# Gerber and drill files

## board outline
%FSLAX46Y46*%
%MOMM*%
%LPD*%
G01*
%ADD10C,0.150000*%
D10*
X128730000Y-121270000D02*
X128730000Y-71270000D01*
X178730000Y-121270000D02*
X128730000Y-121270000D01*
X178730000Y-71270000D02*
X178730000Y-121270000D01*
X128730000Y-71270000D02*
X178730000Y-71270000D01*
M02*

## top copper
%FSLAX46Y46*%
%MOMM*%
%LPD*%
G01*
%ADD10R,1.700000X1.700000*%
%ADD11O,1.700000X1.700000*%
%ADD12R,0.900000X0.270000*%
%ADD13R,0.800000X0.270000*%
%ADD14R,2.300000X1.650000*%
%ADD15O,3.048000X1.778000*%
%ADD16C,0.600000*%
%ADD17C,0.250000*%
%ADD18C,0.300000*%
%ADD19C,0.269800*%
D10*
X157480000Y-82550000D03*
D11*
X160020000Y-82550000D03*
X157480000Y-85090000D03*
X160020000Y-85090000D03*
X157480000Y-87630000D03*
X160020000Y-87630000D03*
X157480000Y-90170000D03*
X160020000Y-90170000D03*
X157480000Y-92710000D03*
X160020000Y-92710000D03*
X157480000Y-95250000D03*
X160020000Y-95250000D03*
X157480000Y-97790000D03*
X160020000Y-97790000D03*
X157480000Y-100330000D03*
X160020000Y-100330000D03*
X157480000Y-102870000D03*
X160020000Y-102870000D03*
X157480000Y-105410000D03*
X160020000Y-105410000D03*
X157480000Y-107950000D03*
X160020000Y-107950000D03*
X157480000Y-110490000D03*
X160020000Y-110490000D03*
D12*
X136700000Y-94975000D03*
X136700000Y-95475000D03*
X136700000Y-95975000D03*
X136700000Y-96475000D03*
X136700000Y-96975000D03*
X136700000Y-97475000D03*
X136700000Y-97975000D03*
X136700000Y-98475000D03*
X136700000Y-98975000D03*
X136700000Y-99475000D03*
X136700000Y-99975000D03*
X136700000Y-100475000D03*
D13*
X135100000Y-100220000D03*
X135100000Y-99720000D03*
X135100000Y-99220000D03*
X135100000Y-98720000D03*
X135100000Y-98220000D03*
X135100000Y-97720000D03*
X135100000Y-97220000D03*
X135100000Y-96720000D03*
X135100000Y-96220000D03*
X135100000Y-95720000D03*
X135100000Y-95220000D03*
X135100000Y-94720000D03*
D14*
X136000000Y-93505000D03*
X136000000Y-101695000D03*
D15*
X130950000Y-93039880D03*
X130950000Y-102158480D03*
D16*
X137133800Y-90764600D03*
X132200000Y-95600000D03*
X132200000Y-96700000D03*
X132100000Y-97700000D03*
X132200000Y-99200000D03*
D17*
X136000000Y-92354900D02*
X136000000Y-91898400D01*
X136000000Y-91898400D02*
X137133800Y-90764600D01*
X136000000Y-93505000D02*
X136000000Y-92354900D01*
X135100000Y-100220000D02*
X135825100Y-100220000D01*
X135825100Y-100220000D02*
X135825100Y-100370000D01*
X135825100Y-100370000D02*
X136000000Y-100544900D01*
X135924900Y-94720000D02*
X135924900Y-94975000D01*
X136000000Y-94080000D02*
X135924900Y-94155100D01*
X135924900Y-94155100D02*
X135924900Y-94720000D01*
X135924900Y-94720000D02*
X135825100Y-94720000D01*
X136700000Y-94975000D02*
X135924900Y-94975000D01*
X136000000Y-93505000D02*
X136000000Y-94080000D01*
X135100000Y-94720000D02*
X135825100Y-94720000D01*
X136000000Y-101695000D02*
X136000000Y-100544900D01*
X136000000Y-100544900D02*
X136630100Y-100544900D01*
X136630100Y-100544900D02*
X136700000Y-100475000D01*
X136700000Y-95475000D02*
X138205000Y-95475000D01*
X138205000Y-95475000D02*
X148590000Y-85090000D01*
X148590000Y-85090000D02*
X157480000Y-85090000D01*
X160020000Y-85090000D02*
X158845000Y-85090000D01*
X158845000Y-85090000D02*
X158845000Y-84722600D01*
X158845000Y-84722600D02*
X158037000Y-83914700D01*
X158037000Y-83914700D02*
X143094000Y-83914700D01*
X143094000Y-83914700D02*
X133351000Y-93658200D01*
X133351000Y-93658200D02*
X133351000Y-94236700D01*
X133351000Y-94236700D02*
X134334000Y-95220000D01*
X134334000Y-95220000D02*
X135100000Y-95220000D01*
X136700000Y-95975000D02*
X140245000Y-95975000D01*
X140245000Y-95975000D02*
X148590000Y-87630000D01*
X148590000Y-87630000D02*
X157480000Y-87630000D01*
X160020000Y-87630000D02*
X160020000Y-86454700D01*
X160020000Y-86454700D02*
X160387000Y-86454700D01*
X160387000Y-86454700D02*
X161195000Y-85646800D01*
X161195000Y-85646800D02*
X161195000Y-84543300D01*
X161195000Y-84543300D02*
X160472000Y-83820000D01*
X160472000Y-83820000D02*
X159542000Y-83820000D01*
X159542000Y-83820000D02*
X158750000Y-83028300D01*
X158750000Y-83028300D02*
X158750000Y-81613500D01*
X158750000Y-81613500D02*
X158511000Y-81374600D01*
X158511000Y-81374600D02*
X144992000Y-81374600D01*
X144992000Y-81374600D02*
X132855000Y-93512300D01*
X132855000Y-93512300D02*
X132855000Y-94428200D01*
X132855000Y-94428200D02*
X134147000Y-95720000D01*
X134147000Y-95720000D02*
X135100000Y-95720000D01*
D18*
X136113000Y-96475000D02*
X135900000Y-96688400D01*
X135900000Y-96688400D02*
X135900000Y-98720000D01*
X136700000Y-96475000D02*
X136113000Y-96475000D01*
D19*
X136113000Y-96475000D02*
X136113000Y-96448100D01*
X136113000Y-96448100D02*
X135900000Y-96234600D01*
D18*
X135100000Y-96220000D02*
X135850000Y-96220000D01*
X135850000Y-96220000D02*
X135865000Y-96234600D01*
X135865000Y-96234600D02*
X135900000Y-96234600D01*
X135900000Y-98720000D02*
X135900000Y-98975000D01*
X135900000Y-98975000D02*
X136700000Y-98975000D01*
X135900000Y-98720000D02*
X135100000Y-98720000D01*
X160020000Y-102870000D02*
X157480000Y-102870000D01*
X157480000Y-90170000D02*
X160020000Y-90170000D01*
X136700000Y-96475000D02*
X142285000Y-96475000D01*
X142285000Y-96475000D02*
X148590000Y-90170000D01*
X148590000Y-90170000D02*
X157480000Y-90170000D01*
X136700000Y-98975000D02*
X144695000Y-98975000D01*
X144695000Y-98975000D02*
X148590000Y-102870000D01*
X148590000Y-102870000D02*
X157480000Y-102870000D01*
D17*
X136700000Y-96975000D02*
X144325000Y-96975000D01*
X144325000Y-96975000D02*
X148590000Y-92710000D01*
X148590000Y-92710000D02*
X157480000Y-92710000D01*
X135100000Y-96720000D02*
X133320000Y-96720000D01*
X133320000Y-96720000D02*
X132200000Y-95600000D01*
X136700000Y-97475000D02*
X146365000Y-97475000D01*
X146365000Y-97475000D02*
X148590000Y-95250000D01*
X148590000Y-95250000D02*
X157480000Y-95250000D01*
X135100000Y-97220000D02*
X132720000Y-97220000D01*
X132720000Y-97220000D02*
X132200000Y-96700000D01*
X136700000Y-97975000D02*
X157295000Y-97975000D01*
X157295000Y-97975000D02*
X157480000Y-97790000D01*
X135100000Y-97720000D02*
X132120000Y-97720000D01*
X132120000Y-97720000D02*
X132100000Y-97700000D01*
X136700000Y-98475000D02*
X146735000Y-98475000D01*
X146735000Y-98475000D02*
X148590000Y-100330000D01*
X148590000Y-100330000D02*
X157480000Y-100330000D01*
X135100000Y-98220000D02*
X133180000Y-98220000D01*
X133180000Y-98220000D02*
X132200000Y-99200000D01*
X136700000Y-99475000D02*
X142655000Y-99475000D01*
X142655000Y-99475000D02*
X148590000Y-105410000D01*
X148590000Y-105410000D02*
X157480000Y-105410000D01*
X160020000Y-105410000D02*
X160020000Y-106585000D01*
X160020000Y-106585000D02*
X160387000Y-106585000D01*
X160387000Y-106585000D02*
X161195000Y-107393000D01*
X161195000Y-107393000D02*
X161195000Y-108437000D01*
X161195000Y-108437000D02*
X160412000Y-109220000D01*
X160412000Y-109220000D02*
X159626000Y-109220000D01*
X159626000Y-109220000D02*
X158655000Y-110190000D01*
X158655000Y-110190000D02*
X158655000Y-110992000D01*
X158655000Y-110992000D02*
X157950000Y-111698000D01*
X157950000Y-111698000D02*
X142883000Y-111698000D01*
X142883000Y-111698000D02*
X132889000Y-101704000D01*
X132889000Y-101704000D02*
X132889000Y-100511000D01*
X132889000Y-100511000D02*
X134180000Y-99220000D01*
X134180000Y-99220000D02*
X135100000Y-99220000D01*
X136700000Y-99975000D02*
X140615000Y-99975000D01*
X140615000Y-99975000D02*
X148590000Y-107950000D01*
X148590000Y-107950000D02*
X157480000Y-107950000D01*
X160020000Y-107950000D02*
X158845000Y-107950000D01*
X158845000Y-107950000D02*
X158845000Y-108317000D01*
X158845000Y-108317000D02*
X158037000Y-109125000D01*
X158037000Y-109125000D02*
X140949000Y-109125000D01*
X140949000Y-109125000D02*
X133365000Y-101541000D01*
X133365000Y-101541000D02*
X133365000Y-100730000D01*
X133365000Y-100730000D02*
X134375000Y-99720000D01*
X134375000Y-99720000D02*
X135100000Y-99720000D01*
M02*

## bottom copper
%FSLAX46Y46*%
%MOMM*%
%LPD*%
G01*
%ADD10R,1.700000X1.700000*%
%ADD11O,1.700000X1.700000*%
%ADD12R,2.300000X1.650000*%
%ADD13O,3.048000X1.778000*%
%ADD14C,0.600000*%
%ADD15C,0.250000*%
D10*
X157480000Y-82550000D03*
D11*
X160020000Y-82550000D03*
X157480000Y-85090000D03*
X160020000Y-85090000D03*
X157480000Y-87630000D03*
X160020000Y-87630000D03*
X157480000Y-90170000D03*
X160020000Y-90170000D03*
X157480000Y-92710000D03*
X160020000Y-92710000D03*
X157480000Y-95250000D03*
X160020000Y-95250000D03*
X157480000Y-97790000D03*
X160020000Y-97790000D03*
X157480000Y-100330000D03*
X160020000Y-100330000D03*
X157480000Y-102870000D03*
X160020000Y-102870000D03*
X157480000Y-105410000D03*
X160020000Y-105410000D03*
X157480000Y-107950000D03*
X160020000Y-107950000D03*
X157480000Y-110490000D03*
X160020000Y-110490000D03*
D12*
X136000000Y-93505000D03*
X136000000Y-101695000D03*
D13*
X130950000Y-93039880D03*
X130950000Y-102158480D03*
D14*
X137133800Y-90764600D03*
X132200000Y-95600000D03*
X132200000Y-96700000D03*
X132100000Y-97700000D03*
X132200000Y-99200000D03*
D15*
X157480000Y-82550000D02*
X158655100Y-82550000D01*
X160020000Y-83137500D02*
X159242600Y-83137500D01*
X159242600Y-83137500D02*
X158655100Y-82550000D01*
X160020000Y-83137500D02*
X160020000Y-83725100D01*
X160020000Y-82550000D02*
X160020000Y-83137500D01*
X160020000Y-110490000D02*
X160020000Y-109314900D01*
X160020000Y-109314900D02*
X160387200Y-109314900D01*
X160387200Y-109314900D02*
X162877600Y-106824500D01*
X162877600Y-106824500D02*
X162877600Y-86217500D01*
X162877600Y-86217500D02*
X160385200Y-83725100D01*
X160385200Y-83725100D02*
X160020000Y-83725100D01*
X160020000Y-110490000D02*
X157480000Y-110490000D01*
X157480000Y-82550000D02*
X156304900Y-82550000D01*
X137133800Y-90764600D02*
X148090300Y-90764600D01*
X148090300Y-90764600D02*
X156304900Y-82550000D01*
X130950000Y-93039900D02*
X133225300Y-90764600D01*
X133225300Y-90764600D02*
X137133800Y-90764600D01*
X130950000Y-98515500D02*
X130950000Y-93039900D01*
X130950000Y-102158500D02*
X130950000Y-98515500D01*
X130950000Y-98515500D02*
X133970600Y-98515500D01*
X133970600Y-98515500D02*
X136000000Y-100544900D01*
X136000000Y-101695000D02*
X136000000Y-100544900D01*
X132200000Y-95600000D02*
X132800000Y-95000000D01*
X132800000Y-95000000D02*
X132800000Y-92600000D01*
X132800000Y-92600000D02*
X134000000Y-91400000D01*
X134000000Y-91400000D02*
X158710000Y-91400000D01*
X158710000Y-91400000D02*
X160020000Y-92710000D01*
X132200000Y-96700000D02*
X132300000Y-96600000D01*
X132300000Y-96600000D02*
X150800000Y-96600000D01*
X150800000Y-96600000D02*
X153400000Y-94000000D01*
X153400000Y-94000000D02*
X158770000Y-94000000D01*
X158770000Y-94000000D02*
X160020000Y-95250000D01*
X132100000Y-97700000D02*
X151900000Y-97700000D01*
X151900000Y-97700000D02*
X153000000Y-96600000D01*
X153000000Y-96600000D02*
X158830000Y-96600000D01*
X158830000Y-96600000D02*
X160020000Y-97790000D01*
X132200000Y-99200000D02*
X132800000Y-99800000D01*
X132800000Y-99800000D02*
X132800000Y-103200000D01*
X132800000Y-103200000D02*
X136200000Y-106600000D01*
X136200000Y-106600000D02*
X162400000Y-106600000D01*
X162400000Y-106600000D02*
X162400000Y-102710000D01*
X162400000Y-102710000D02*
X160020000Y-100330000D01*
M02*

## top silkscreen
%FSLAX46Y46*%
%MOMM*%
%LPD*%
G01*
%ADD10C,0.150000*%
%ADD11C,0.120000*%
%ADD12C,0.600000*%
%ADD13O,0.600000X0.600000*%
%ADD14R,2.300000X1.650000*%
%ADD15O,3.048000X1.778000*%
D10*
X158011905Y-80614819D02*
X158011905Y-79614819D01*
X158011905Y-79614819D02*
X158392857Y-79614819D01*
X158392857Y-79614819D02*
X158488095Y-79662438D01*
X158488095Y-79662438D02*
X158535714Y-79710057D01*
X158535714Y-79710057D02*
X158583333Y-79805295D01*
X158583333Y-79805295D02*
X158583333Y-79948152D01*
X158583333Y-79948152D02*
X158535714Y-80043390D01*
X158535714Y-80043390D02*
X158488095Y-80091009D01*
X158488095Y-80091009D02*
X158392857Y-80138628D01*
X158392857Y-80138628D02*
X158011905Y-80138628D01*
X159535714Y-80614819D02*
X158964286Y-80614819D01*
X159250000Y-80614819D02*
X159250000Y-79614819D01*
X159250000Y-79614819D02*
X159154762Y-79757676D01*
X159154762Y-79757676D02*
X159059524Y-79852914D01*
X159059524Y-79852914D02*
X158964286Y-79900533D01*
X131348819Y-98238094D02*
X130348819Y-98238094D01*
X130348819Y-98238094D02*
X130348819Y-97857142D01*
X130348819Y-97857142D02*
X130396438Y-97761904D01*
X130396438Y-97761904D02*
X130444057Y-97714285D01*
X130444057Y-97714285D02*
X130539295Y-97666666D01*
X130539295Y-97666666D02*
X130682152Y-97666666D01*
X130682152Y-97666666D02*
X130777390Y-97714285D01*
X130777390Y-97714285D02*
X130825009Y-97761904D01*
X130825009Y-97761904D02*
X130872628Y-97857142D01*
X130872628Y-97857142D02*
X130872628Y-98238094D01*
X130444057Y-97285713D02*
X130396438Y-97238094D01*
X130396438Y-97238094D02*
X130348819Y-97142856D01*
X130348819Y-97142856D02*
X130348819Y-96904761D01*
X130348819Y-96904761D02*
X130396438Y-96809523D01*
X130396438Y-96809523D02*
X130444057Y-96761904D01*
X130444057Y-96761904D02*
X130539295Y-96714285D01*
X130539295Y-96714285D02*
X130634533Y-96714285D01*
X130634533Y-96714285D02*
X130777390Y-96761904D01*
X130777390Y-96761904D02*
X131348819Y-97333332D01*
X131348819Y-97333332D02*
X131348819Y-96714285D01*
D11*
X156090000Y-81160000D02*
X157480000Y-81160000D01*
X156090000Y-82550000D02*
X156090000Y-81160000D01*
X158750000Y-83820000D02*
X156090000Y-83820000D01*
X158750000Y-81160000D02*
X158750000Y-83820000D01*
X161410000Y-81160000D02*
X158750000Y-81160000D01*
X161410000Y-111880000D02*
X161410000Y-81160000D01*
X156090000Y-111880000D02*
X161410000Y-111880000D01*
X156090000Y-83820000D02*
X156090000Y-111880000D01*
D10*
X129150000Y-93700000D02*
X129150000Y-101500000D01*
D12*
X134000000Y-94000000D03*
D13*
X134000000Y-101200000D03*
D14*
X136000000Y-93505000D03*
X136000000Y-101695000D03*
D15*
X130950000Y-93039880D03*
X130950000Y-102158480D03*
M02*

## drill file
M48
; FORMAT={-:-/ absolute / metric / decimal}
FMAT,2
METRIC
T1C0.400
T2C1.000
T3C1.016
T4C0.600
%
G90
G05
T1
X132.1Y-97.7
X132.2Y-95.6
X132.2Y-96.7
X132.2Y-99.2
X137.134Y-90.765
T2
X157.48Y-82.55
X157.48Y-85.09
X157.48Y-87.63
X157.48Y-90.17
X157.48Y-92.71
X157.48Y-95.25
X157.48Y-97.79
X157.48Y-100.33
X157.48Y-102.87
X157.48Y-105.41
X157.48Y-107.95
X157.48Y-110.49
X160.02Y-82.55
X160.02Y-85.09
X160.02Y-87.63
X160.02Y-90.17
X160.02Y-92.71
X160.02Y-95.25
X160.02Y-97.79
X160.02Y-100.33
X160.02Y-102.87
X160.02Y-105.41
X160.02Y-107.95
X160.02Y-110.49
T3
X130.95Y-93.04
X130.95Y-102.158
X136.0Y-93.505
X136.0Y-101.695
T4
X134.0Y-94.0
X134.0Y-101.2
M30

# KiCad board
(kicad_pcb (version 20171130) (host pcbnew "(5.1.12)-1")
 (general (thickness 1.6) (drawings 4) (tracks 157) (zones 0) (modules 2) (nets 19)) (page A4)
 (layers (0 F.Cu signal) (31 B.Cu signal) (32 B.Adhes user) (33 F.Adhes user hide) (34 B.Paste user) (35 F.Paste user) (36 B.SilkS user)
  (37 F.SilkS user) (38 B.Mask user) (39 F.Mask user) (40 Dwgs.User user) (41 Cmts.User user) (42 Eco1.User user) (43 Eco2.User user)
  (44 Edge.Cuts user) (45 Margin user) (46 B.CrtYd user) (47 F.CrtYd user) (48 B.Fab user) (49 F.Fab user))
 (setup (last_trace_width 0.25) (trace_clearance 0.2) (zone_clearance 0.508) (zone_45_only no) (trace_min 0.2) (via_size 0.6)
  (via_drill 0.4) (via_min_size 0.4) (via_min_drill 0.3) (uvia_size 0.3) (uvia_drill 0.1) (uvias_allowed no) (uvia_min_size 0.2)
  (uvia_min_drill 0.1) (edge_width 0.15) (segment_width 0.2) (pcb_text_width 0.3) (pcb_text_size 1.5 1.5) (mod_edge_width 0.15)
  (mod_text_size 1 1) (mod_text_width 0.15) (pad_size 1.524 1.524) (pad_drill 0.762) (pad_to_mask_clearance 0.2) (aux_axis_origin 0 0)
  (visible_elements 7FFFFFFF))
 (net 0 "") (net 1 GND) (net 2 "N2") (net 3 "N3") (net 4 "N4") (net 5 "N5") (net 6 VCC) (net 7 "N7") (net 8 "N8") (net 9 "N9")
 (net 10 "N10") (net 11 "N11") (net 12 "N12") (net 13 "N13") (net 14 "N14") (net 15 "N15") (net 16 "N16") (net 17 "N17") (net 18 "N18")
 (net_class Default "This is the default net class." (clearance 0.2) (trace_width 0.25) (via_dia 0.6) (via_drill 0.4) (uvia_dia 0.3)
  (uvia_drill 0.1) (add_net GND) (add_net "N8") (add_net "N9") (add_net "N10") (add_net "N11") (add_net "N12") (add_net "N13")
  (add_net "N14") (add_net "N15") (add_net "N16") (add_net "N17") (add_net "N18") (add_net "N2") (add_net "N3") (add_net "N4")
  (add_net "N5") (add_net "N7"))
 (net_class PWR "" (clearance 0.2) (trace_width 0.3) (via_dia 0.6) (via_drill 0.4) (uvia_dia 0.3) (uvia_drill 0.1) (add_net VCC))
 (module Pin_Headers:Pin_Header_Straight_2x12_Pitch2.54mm (layer F.Cu) (at 157.48 82.55)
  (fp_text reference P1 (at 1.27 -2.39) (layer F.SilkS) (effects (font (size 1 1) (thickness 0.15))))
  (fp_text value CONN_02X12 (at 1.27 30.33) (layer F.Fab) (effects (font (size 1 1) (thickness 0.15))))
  (fp_line (start -1.39 -1.39) (end 0 -1.39) (layer F.SilkS) (width 0.12))
  (fp_line (start -1.39 0) (end -1.39 -1.39) (layer F.SilkS) (width 0.12))
  (fp_line (start 1.27 1.27) (end -1.39 1.27) (layer F.SilkS) (width 0.12))
  (fp_line (start 1.27 -1.39) (end 1.27 1.27) (layer F.SilkS) (width 0.12))
  (fp_line (start 3.93 -1.39) (end 1.27 -1.39) (layer F.SilkS) (width 0.12))
  (fp_line (start 3.93 29.33) (end 3.93 -1.39) (layer F.SilkS) (width 0.12))
  (fp_line (start -1.39 29.33) (end 3.93 29.33) (layer F.SilkS) (width 0.12))
  (fp_line (start -1.39 1.27) (end -1.39 29.33) (layer F.SilkS) (width 0.12))
  (pad 1 thru_hole rect (at 0 0) (size 1.7 1.7) (drill 1) (layers *.Cu *.Mask) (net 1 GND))
  (pad 2 thru_hole oval (at 2.54 0) (size 1.7 1.7) (drill 1) (layers *.Cu *.Mask) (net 1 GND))
  (pad 3 thru_hole oval (at 0 2.54) (size 1.7 1.7) (drill 1) (layers *.Cu *.Mask) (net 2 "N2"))
  (pad 4 thru_hole oval (at 2.54 2.54) (size 1.7 1.7) (drill 1) (layers *.Cu *.Mask) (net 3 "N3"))
  (pad 5 thru_hole oval (at 0 5.08) (size 1.7 1.7) (drill 1) (layers *.Cu *.Mask) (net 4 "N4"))
  (pad 6 thru_hole oval (at 2.54 5.08) (size 1.7 1.7) (drill 1) (layers *.Cu *.Mask) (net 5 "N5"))
  (pad 7 thru_hole oval (at 0 7.62) (size 1.7 1.7) (drill 1) (layers *.Cu *.Mask) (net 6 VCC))
  (pad 8 thru_hole oval (at 2.54 7.62) (size 1.7 1.7) (drill 1) (layers *.Cu *.Mask) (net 6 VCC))
  (pad 9 thru_hole oval (at 0 10.16) (size 1.7 1.7) (drill 1) (layers *.Cu *.Mask) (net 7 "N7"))
  (pad 10 thru_hole oval (at 2.54 10.16) (size 1.7 1.7) (drill 1) (layers *.Cu *.Mask) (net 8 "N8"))
  (pad 11 thru_hole oval (at 0 12.7) (size 1.7 1.7) (drill 1) (layers *.Cu *.Mask) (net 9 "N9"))
  (pad 12 thru_hole oval (at 2.54 12.7) (size 1.7 1.7) (drill 1) (layers *.Cu *.Mask) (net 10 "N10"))
  (pad 13 thru_hole oval (at 0 15.24) (size 1.7 1.7) (drill 1) (layers *.Cu *.Mask) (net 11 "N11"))
  (pad 14 thru_hole oval (at 2.54 15.24) (size 1.7 1.7) (drill 1) (layers *.Cu *.Mask) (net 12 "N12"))
  (pad 15 thru_hole oval (at 0 17.78) (size 1.7 1.7) (drill 1) (layers *.Cu *.Mask) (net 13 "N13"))
  (pad 16 thru_hole oval (at 2.54 17.78) (size 1.7 1.7) (drill 1) (layers *.Cu *.Mask) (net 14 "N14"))
  (pad 17 thru_hole oval (at 0 20.32) (size 1.7 1.7) (drill 1) (layers *.Cu *.Mask) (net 6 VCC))
  (pad 18 thru_hole oval (at 2.54 20.32) (size 1.7 1.7) (drill 1) (layers *.Cu *.Mask) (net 6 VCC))
  (pad 19 thru_hole oval (at 0 22.86) (size 1.7 1.7) (drill 1) (layers *.Cu *.Mask) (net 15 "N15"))
  (pad 20 thru_hole oval (at 2.54 22.86) (size 1.7 1.7) (drill 1) (layers *.Cu *.Mask) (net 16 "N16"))
  (pad 21 thru_hole oval (at 0 25.4) (size 1.7 1.7) (drill 1) (layers *.Cu *.Mask) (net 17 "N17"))
  (pad 22 thru_hole oval (at 2.54 25.4) (size 1.7 1.7) (drill 1) (layers *.Cu *.Mask) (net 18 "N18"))
  (pad 23 thru_hole oval (at 0 27.94) (size 1.7 1.7) (drill 1) (layers *.Cu *.Mask) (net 1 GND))
  (pad 24 thru_hole oval (at 2.54 27.94) (size 1.7 1.7) (drill 1) (layers *.Cu *.Mask) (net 1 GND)))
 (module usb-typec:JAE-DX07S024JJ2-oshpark (layer F.Cu) (at 134 94 270)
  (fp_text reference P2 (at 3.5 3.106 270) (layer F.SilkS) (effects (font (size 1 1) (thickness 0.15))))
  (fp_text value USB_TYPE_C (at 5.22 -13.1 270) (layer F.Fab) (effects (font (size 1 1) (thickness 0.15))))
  (fp_line (start -0.3 4.85) (end 7.5 4.85) (layer F.SilkS) (width 0.15))
  (pad A1 smd rect (at 0.975 -2.7 270) (size 0.27 0.9) (layers F.Cu F.Paste F.Mask) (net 1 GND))
  (pad A2 smd rect (at 1.475 -2.7 270) (size 0.27 0.9) (layers F.Cu F.Paste F.Mask) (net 2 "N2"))
  (pad A3 smd rect (at 1.975 -2.7 270) (size 0.27 0.9) (layers F.Cu F.Paste F.Mask) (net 4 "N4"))
  (pad A4 smd rect (at 2.475 -2.7 270) (size 0.27 0.9) (layers F.Cu F.Paste F.Mask) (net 6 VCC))
  (pad A5 smd rect (at 2.975 -2.7 270) (size 0.27 0.9) (layers F.Cu F.Paste F.Mask) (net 7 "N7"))
  (pad A6 smd rect (at 3.475 -2.7 270) (size 0.27 0.9) (layers F.Cu F.Paste F.Mask) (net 9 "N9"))
  (pad A7 smd rect (at 3.975 -2.7 270) (size 0.27 0.9) (layers F.Cu F.Paste F.Mask) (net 11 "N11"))
  (pad A8 smd rect (at 4.475 -2.7 270) (size 0.27 0.9) (layers F.Cu F.Paste F.Mask) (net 13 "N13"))
  (pad A9 smd rect (at 4.975 -2.7 270) (size 0.27 0.9) (layers F.Cu F.Paste F.Mask) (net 6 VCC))
  (pad A10 smd rect (at 5.475 -2.7 270) (size 0.27 0.9) (layers F.Cu F.Paste F.Mask) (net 15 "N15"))
  (pad A11 smd rect (at 5.975 -2.7 270) (size 0.27 0.9) (layers F.Cu F.Paste F.Mask) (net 17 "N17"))
  (pad A12 smd rect (at 6.475 -2.7 270) (size 0.27 0.9) (layers F.Cu F.Paste F.Mask) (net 1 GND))
  (pad B1 smd rect (at 6.22 -1.1 270) (size 0.27 0.8) (layers F.Cu F.Paste F.Mask) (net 1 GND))
  (pad B2 smd rect (at 5.72 -1.1 270) (size 0.27 0.8) (layers F.Cu F.Paste F.Mask) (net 18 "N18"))
  (pad B3 smd rect (at 5.22 -1.1 270) (size 0.27 0.8) (layers F.Cu F.Paste F.Mask) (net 16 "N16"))
  (pad B4 smd rect (at 4.72 -1.1 270) (size 0.27 0.8) (layers F.Cu F.Paste F.Mask) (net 6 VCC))
  (pad B5 smd rect (at 4.22 -1.1 270) (size 0.27 0.8) (layers F.Cu F.Paste F.Mask) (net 14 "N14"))
  (pad B6 smd rect (at 3.72 -1.1 270) (size 0.27 0.8) (layers F.Cu F.Paste F.Mask) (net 12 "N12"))
  (pad B7 smd rect (at 3.22 -1.1 270) (size 0.27 0.8) (layers F.Cu F.Paste F.Mask) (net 10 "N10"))
  (pad B8 smd rect (at 2.72 -1.1 270) (size 0.27 0.8) (layers F.Cu F.Paste F.Mask) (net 8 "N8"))
  (pad B9 smd rect (at 2.22 -1.1 270) (size 0.27 0.8) (layers F.Cu F.Paste F.Mask) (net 6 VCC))
  (pad B10 smd rect (at 1.72 -1.1 270) (size 0.27 0.8) (layers F.Cu F.Paste F.Mask) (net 5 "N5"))
  (pad B11 smd rect (at 1.22 -1.1 270) (size 0.27 0.8) (layers F.Cu F.Paste F.Mask) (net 3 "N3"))
  (pad B12 smd rect (at 0.72 -1.1 270) (size 0.27 0.8) (layers F.Cu F.Paste F.Mask) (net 1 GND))
  (pad "" np_thru_hole circle (at 0 0 270) (size 0.6 0.6) (drill 0.6) (layers *.Cu *.Mask F.SilkS))
  (pad "" np_thru_hole oval (at 7.2 0 270) (size 0.6 0.6) (drill 0.6) (layers *.Cu *.Mask F.SilkS))
  (pad 0 thru_hole rect (at -0.495 -2 270) (size 1.65 2.3) (drill 1.016) (layers *.Cu *.Mask F.SilkS) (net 1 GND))
  (pad 0 thru_hole rect (at 7.695 -2 270) (size 1.65 2.3) (drill 1.016) (layers *.Cu *.Mask F.SilkS) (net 1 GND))
  (pad 0 thru_hole oval (at -0.96012 3.05 270) (size 1.778 3.048) (drill 1.016) (layers *.Cu *.Mask F.SilkS) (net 1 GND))
  (pad 0 thru_hole oval (at 8.15848 3.05 270) (size 1.778 3.048) (drill 1.016) (layers *.Cu *.Mask F.SilkS) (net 1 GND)))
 (gr_line (start 128.73 121.27) (end 128.73 71.27) (angle 90) (layer Edge.Cuts) (width 0.15))
 (gr_line (start 178.73 121.27) (end 128.73 121.27) (angle 90) (layer Edge.Cuts) (width 0.15))
 (gr_line (start 178.73 71.27) (end 178.73 121.27) (angle 90) (layer Edge.Cuts) (width 0.15))
 (gr_line (start 128.73 71.27) (end 178.73 71.27) (angle 90) (layer Edge.Cuts) (width 0.15))
 (segment (start 157.48 82.55) (end 158.6551 82.55) (width 0.25) (layer B.Cu) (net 1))
 (segment (start 160.02 83.1375) (end 159.2426 83.1375) (width 0.25) (layer B.Cu) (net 1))
 (segment (start 159.2426 83.1375) (end 158.6551 82.55) (width 0.25) (layer B.Cu) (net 1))
 (segment (start 160.02 83.1375) (end 160.02 83.7251) (width 0.25) (layer B.Cu) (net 1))
 (segment (start 160.02 82.55) (end 160.02 83.1375) (width 0.25) (layer B.Cu) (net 1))
 (segment (start 160.02 110.49) (end 160.02 109.3149) (width 0.25) (layer B.Cu) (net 1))
 (segment (start 160.02 109.3149) (end 160.3872 109.3149) (width 0.25) (layer B.Cu) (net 1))
 (segment (start 160.3872 109.3149) (end 162.8776 106.8245) (width 0.25) (layer B.Cu) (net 1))
 (segment (start 162.8776 106.8245) (end 162.8776 86.2175) (width 0.25) (layer B.Cu) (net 1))
 (segment (start 162.8776 86.2175) (end 160.3852 83.7251) (width 0.25) (layer B.Cu) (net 1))
 (segment (start 160.3852 83.7251) (end 160.02 83.7251) (width 0.25) (layer B.Cu) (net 1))
 (segment (start 160.02 110.49) (end 157.48 110.49) (width 0.25) (layer B.Cu) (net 1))
 (segment (start 157.48 82.55) (end 156.3049 82.55) (width 0.25) (layer B.Cu) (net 1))
 (segment (start 137.1338 90.7646) (end 148.0903 90.7646) (width 0.25) (layer B.Cu) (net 1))
 (segment (start 148.0903 90.7646) (end 156.3049 82.55) (width 0.25) (layer B.Cu) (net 1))
 (segment (start 130.95 93.0399) (end 133.2253 90.7646) (width 0.25) (layer B.Cu) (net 1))
 (segment (start 133.2253 90.7646) (end 137.1338 90.7646) (width 0.25) (layer B.Cu) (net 1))
 (segment (start 136 92.3549) (end 136 91.8984) (width 0.25) (layer F.Cu) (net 1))
 (segment (start 136 91.8984) (end 137.1338 90.7646) (width 0.25) (layer F.Cu) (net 1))
 (segment (start 136 93.505) (end 136 92.3549) (width 0.25) (layer F.Cu) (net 1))
 (segment (start 130.95 98.5155) (end 130.95 93.0399) (width 0.25) (layer B.Cu) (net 1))
 (segment (start 135.1 100.22) (end 135.8251 100.22) (width 0.25) (layer F.Cu) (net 1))
 (segment (start 135.8251 100.22) (end 135.8251 100.37) (width 0.25) (layer F.Cu) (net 1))
 (segment (start 135.8251 100.37) (end 136 100.5449) (width 0.25) (layer F.Cu) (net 1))
 (segment (start 135.9249 94.72) (end 135.9249 94.975) (width 0.25) (layer F.Cu) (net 1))
 (segment (start 136 94.08) (end 135.9249 94.1551) (width 0.25) (layer F.Cu) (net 1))
 (segment (start 135.9249 94.1551) (end 135.9249 94.72) (width 0.25) (layer F.Cu) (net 1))
 (segment (start 135.9249 94.72) (end 135.8251 94.72) (width 0.25) (layer F.Cu) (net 1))
 (segment (start 136.7 94.975) (end 135.9249 94.975) (width 0.25) (layer F.Cu) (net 1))
 (segment (start 136 93.505) (end 136 94.08) (width 0.25) (layer F.Cu) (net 1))
 (segment (start 135.1 94.72) (end 135.8251 94.72) (width 0.25) (layer F.Cu) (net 1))
 (segment (start 136 101.695) (end 136 100.5449) (width 0.25) (layer F.Cu) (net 1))
 (segment (start 136 100.5449) (end 136.6301 100.5449) (width 0.25) (layer F.Cu) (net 1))
 (segment (start 136.6301 100.5449) (end 136.7 100.475) (width 0.25) (layer F.Cu) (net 1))
 (segment (start 130.95 102.1585) (end 130.95 98.5155) (width 0.25) (layer B.Cu) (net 1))
 (segment (start 130.95 98.5155) (end 133.9706 98.5155) (width 0.25) (layer B.Cu) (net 1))
 (segment (start 133.9706 98.5155) (end 136 100.5449) (width 0.25) (layer B.Cu) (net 1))
 (segment (start 136 101.695) (end 136 100.5449) (width 0.25) (layer B.Cu) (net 1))
 (via (at 137.1338 90.7646) (size 0.6) (layers F.Cu B.Cu) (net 1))
 (segment (start 136.7 95.475) (end 138.205 95.475) (width 0.25) (layer F.Cu) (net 2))
 (segment (start 138.205 95.475) (end 148.59 85.09) (width 0.25) (layer F.Cu) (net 2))
 (segment (start 148.59 85.09) (end 157.48 85.09) (width 0.25) (layer F.Cu) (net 2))
 (segment (start 160.02 85.09) (end 158.845 85.09) (width 0.25) (layer F.Cu) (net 3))
 (segment (start 158.845 85.09) (end 158.845 84.7226) (width 0.25) (layer F.Cu) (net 3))
 (segment (start 158.845 84.7226) (end 158.037 83.9147) (width 0.25) (layer F.Cu) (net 3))
 (segment (start 158.037 83.9147) (end 143.094 83.9147) (width 0.25) (layer F.Cu) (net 3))
 (segment (start 143.094 83.9147) (end 133.351 93.6582) (width 0.25) (layer F.Cu) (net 3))
 (segment (start 133.351 93.6582) (end 133.351 94.2367) (width 0.25) (layer F.Cu) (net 3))
 (segment (start 133.351 94.2367) (end 134.334 95.22) (width 0.25) (layer F.Cu) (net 3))
 (segment (start 134.334 95.22) (end 135.1 95.22) (width 0.25) (layer F.Cu) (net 3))
 (segment (start 136.7 95.975) (end 140.245 95.975) (width 0.25) (layer F.Cu) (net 4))
 (segment (start 140.245 95.975) (end 148.59 87.63) (width 0.25) (layer F.Cu) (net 4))
 (segment (start 148.59 87.63) (end 157.48 87.63) (width 0.25) (layer F.Cu) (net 4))
 (segment (start 160.02 87.63) (end 160.02 86.4547) (width 0.25) (layer F.Cu) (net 5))
 (segment (start 160.02 86.4547) (end 160.387 86.4547) (width 0.25) (layer F.Cu) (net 5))
 (segment (start 160.387 86.4547) (end 161.195 85.6468) (width 0.25) (layer F.Cu) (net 5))
 (segment (start 161.195 85.6468) (end 161.195 84.5433) (width 0.25) (layer F.Cu) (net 5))
 (segment (start 161.195 84.5433) (end 160.472 83.82) (width 0.25) (layer F.Cu) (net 5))
 (segment (start 160.472 83.82) (end 159.542 83.82) (width 0.25) (layer F.Cu) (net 5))
 (segment (start 159.542 83.82) (end 158.75 83.0283) (width 0.25) (layer F.Cu) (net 5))
 (segment (start 158.75 83.0283) (end 158.75 81.6135) (width 0.25) (layer F.Cu) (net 5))
 (segment (start 158.75 81.6135) (end 158.511 81.3746) (width 0.25) (layer F.Cu) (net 5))
 (segment (start 158.511 81.3746) (end 144.992 81.3746) (width 0.25) (layer F.Cu) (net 5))
 (segment (start 144.992 81.3746) (end 132.855 93.5123) (width 0.25) (layer F.Cu) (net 5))
 (segment (start 132.855 93.5123) (end 132.855 94.4282) (width 0.25) (layer F.Cu) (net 5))
 (segment (start 132.855 94.4282) (end 134.147 95.72) (width 0.25) (layer F.Cu) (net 5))
 (segment (start 134.147 95.72) (end 135.1 95.72) (width 0.25) (layer F.Cu) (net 5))
 (segment (start 136.113 96.475) (end 135.9 96.6884) (width 0.3) (layer F.Cu) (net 6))
 (segment (start 135.9 96.6884) (end 135.9 98.72) (width 0.3) (layer F.Cu) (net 6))
 (segment (start 136.7 96.475) (end 136.113 96.475) (width 0.3) (layer F.Cu) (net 6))
 (segment (start 136.113 96.475) (end 136.113 96.4481) (width 0.2698) (layer F.Cu) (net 6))
 (segment (start 136.113 96.4481) (end 135.9 96.2346) (width 0.2698) (layer F.Cu) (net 6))
 (segment (start 135.1 96.22) (end 135.85 96.22) (width 0.3) (layer F.Cu) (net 6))
 (segment (start 135.85 96.22) (end 135.865 96.2346) (width 0.3) (layer F.Cu) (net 6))
 (segment (start 135.865 96.2346) (end 135.9 96.2346) (width 0.3) (layer F.Cu) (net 6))
 (segment (start 135.9 98.72) (end 135.9 98.975) (width 0.3) (layer F.Cu) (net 6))
 (segment (start 135.9 98.975) (end 136.7 98.975) (width 0.3) (layer F.Cu) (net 6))
 (segment (start 135.9 98.72) (end 135.1 98.72) (width 0.3) (layer F.Cu) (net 6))
 (segment (start 160.02 102.87) (end 157.48 102.87) (width 0.3) (layer F.Cu) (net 6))
 (segment (start 157.48 90.17) (end 160.02 90.17) (width 0.3) (layer F.Cu) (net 6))
 (segment (start 136.7 96.475) (end 142.285 96.475) (width 0.3) (layer F.Cu) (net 6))
 (segment (start 142.285 96.475) (end 148.59 90.17) (width 0.3) (layer F.Cu) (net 6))
 (segment (start 148.59 90.17) (end 157.48 90.17) (width 0.3) (layer F.Cu) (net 6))
 (segment (start 136.7 98.975) (end 144.695 98.975) (width 0.3) (layer F.Cu) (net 6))
 (segment (start 144.695 98.975) (end 148.59 102.87) (width 0.3) (layer F.Cu) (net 6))
 (segment (start 148.59 102.87) (end 157.48 102.87) (width 0.3) (layer F.Cu) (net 6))
 (segment (start 136.7 96.975) (end 144.325 96.975) (width 0.25) (layer F.Cu) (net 7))
 (segment (start 144.325 96.975) (end 148.59 92.71) (width 0.25) (layer F.Cu) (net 7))
 (segment (start 148.59 92.71) (end 157.48 92.71) (width 0.25) (layer F.Cu) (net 7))
 (segment (start 135.1 96.72) (end 133.32 96.72) (width 0.25) (layer F.Cu) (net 8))
 (segment (start 133.32 96.72) (end 132.2 95.6) (width 0.25) (layer F.Cu) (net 8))
 (segment (start 132.2 95.6) (end 132.8 95) (width 0.25) (layer B.Cu) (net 8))
 (segment (start 132.8 95) (end 132.8 92.6) (width 0.25) (layer B.Cu) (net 8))
 (segment (start 132.8 92.6) (end 134 91.4) (width 0.25) (layer B.Cu) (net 8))
 (segment (start 134 91.4) (end 158.71 91.4) (width 0.25) (layer B.Cu) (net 8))
 (segment (start 158.71 91.4) (end 160.02 92.71) (width 0.25) (layer B.Cu) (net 8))
 (via (at 132.2 95.6) (size 0.6) (layers F.Cu B.Cu) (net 8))
 (segment (start 136.7 97.475) (end 146.365 97.475) (width 0.25) (layer F.Cu) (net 9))
 (segment (start 146.365 97.475) (end 148.59 95.25) (width 0.25) (layer F.Cu) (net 9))
 (segment (start 148.59 95.25) (end 157.48 95.25) (width 0.25) (layer F.Cu) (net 9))
 (segment (start 135.1 97.22) (end 132.72 97.22) (width 0.25) (layer F.Cu) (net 10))
 (segment (start 132.72 97.22) (end 132.2 96.7) (width 0.25) (layer F.Cu) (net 10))
 (segment (start 132.2 96.7) (end 132.3 96.6) (width 0.25) (layer B.Cu) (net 10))
 (segment (start 132.3 96.6) (end 150.8 96.6) (width 0.25) (layer B.Cu) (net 10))
 (segment (start 150.8 96.6) (end 153.4 94) (width 0.25) (layer B.Cu) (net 10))
 (segment (start 153.4 94) (end 158.77 94) (width 0.25) (layer B.Cu) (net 10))
 (segment (start 158.77 94) (end 160.02 95.25) (width 0.25) (layer B.Cu) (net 10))
 (via (at 132.2 96.7) (size 0.6) (layers F.Cu B.Cu) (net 10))
 (segment (start 136.7 97.975) (end 157.295 97.975) (width 0.25) (layer F.Cu) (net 11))
 (segment (start 157.295 97.975) (end 157.48 97.79) (width 0.25) (layer F.Cu) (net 11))
 (segment (start 135.1 97.72) (end 132.12 97.72) (width 0.25) (layer F.Cu) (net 12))
 (segment (start 132.12 97.72) (end 132.1 97.7) (width 0.25) (layer F.Cu) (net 12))
 (segment (start 132.1 97.7) (end 151.9 97.7) (width 0.25) (layer B.Cu) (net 12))
 (segment (start 151.9 97.7) (end 153 96.6) (width 0.25) (layer B.Cu) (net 12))
 (segment (start 153 96.6) (end 158.83 96.6) (width 0.25) (layer B.Cu) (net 12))
 (segment (start 158.83 96.6) (end 160.02 97.79) (width 0.25) (layer B.Cu) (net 12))
 (via (at 132.1 97.7) (size 0.6) (layers F.Cu B.Cu) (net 12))
 (segment (start 136.7 98.475) (end 146.735 98.475) (width 0.25) (layer F.Cu) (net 13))
 (segment (start 146.735 98.475) (end 148.59 100.33) (width 0.25) (layer F.Cu) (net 13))
 (segment (start 148.59 100.33) (end 157.48 100.33) (width 0.25) (layer F.Cu) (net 13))
 (segment (start 132.2 99.2) (end 132.8 99.8) (width 0.25) (layer B.Cu) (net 14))
 (segment (start 132.8 99.8) (end 132.8 103.2) (width 0.25) (layer B.Cu) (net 14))
 (segment (start 132.8 103.2) (end 136.2 106.6) (width 0.25) (layer B.Cu) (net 14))
 (segment (start 136.2 106.6) (end 162.4 106.6) (width 0.25) (layer B.Cu) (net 14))
 (segment (start 162.4 106.6) (end 162.4 102.71) (width 0.25) (layer B.Cu) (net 14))
 (segment (start 162.4 102.71) (end 160.02 100.33) (width 0.25) (layer B.Cu) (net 14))
 (segment (start 135.1 98.22) (end 133.18 98.22) (width 0.25) (layer F.Cu) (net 14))
 (segment (start 133.18 98.22) (end 132.2 99.2) (width 0.25) (layer F.Cu) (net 14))
 (via (at 132.2 99.2) (size 0.6) (layers F.Cu B.Cu) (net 14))
 (segment (start 136.7 99.475) (end 142.655 99.475) (width 0.25) (layer F.Cu) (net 15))
 (segment (start 142.655 99.475) (end 148.59 105.41) (width 0.25) (layer F.Cu) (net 15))
 (segment (start 148.59 105.41) (end 157.48 105.41) (width 0.25) (layer F.Cu) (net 15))
 (segment (start 160.02 105.41) (end 160.02 106.585) (width 0.25) (layer F.Cu) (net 16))
 (segment (start 160.02 106.585) (end 160.387 106.585) (width 0.25) (layer F.Cu) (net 16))
 (segment (start 160.387 106.585) (end 161.195 107.393) (width 0.25) (layer F.Cu) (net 16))
 (segment (start 161.195 107.393) (end 161.195 108.437) (width 0.25) (layer F.Cu) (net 16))
 (segment (start 161.195 108.437) (end 160.412 109.22) (width 0.25) (layer F.Cu) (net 16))
 (segment (start 160.412 109.22) (end 159.626 109.22) (width 0.25) (layer F.Cu) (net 16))
 (segment (start 159.626 109.22) (end 158.655 110.19) (width 0.25) (layer F.Cu) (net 16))
 (segment (start 158.655 110.19) (end 158.655 110.992) (width 0.25) (layer F.Cu) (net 16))
 (segment (start 158.655 110.992) (end 157.95 111.698) (width 0.25) (layer F.Cu) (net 16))
 (segment (start 157.95 111.698) (end 142.883 111.698) (width 0.25) (layer F.Cu) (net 16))
 (segment (start 142.883 111.698) (end 132.889 101.704) (width 0.25) (layer F.Cu) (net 16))
 (segment (start 132.889 101.704) (end 132.889 100.511) (width 0.25) (layer F.Cu) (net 16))
 (segment (start 132.889 100.511) (end 134.18 99.22) (width 0.25) (layer F.Cu) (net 16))
 (segment (start 134.18 99.22) (end 135.1 99.22) (width 0.25) (layer F.Cu) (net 16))
 (segment (start 136.7 99.975) (end 140.615 99.975) (width 0.25) (layer F.Cu) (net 17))
 (segment (start 140.615 99.975) (end 148.59 107.95) (width 0.25) (layer F.Cu) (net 17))
 (segment (start 148.59 107.95) (end 157.48 107.95) (width 0.25) (layer F.Cu) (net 17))
 (segment (start 160.02 107.95) (end 158.845 107.95) (width 0.25) (layer F.Cu) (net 18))
 (segment (start 158.845 107.95) (end 158.845 108.317) (width 0.25) (layer F.Cu) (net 18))
 (segment (start 158.845 108.317) (end 158.037 109.125) (width 0.25) (layer F.Cu) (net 18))
 (segment (start 158.037 109.125) (end 140.949 109.125) (width 0.25) (layer F.Cu) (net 18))
 (segment (start 140.949 109.125) (end 133.365 101.541) (width 0.25) (layer F.Cu) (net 18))
 (segment (start 133.365 101.541) (end 133.365 100.73) (width 0.25) (layer F.Cu) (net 18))
 (segment (start 133.365 100.73) (end 134.375 99.72) (width 0.25) (layer F.Cu) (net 18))
 (segment (start 134.375 99.72) (end 135.1 99.72) (width 0.25) (layer F.Cu) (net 18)))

